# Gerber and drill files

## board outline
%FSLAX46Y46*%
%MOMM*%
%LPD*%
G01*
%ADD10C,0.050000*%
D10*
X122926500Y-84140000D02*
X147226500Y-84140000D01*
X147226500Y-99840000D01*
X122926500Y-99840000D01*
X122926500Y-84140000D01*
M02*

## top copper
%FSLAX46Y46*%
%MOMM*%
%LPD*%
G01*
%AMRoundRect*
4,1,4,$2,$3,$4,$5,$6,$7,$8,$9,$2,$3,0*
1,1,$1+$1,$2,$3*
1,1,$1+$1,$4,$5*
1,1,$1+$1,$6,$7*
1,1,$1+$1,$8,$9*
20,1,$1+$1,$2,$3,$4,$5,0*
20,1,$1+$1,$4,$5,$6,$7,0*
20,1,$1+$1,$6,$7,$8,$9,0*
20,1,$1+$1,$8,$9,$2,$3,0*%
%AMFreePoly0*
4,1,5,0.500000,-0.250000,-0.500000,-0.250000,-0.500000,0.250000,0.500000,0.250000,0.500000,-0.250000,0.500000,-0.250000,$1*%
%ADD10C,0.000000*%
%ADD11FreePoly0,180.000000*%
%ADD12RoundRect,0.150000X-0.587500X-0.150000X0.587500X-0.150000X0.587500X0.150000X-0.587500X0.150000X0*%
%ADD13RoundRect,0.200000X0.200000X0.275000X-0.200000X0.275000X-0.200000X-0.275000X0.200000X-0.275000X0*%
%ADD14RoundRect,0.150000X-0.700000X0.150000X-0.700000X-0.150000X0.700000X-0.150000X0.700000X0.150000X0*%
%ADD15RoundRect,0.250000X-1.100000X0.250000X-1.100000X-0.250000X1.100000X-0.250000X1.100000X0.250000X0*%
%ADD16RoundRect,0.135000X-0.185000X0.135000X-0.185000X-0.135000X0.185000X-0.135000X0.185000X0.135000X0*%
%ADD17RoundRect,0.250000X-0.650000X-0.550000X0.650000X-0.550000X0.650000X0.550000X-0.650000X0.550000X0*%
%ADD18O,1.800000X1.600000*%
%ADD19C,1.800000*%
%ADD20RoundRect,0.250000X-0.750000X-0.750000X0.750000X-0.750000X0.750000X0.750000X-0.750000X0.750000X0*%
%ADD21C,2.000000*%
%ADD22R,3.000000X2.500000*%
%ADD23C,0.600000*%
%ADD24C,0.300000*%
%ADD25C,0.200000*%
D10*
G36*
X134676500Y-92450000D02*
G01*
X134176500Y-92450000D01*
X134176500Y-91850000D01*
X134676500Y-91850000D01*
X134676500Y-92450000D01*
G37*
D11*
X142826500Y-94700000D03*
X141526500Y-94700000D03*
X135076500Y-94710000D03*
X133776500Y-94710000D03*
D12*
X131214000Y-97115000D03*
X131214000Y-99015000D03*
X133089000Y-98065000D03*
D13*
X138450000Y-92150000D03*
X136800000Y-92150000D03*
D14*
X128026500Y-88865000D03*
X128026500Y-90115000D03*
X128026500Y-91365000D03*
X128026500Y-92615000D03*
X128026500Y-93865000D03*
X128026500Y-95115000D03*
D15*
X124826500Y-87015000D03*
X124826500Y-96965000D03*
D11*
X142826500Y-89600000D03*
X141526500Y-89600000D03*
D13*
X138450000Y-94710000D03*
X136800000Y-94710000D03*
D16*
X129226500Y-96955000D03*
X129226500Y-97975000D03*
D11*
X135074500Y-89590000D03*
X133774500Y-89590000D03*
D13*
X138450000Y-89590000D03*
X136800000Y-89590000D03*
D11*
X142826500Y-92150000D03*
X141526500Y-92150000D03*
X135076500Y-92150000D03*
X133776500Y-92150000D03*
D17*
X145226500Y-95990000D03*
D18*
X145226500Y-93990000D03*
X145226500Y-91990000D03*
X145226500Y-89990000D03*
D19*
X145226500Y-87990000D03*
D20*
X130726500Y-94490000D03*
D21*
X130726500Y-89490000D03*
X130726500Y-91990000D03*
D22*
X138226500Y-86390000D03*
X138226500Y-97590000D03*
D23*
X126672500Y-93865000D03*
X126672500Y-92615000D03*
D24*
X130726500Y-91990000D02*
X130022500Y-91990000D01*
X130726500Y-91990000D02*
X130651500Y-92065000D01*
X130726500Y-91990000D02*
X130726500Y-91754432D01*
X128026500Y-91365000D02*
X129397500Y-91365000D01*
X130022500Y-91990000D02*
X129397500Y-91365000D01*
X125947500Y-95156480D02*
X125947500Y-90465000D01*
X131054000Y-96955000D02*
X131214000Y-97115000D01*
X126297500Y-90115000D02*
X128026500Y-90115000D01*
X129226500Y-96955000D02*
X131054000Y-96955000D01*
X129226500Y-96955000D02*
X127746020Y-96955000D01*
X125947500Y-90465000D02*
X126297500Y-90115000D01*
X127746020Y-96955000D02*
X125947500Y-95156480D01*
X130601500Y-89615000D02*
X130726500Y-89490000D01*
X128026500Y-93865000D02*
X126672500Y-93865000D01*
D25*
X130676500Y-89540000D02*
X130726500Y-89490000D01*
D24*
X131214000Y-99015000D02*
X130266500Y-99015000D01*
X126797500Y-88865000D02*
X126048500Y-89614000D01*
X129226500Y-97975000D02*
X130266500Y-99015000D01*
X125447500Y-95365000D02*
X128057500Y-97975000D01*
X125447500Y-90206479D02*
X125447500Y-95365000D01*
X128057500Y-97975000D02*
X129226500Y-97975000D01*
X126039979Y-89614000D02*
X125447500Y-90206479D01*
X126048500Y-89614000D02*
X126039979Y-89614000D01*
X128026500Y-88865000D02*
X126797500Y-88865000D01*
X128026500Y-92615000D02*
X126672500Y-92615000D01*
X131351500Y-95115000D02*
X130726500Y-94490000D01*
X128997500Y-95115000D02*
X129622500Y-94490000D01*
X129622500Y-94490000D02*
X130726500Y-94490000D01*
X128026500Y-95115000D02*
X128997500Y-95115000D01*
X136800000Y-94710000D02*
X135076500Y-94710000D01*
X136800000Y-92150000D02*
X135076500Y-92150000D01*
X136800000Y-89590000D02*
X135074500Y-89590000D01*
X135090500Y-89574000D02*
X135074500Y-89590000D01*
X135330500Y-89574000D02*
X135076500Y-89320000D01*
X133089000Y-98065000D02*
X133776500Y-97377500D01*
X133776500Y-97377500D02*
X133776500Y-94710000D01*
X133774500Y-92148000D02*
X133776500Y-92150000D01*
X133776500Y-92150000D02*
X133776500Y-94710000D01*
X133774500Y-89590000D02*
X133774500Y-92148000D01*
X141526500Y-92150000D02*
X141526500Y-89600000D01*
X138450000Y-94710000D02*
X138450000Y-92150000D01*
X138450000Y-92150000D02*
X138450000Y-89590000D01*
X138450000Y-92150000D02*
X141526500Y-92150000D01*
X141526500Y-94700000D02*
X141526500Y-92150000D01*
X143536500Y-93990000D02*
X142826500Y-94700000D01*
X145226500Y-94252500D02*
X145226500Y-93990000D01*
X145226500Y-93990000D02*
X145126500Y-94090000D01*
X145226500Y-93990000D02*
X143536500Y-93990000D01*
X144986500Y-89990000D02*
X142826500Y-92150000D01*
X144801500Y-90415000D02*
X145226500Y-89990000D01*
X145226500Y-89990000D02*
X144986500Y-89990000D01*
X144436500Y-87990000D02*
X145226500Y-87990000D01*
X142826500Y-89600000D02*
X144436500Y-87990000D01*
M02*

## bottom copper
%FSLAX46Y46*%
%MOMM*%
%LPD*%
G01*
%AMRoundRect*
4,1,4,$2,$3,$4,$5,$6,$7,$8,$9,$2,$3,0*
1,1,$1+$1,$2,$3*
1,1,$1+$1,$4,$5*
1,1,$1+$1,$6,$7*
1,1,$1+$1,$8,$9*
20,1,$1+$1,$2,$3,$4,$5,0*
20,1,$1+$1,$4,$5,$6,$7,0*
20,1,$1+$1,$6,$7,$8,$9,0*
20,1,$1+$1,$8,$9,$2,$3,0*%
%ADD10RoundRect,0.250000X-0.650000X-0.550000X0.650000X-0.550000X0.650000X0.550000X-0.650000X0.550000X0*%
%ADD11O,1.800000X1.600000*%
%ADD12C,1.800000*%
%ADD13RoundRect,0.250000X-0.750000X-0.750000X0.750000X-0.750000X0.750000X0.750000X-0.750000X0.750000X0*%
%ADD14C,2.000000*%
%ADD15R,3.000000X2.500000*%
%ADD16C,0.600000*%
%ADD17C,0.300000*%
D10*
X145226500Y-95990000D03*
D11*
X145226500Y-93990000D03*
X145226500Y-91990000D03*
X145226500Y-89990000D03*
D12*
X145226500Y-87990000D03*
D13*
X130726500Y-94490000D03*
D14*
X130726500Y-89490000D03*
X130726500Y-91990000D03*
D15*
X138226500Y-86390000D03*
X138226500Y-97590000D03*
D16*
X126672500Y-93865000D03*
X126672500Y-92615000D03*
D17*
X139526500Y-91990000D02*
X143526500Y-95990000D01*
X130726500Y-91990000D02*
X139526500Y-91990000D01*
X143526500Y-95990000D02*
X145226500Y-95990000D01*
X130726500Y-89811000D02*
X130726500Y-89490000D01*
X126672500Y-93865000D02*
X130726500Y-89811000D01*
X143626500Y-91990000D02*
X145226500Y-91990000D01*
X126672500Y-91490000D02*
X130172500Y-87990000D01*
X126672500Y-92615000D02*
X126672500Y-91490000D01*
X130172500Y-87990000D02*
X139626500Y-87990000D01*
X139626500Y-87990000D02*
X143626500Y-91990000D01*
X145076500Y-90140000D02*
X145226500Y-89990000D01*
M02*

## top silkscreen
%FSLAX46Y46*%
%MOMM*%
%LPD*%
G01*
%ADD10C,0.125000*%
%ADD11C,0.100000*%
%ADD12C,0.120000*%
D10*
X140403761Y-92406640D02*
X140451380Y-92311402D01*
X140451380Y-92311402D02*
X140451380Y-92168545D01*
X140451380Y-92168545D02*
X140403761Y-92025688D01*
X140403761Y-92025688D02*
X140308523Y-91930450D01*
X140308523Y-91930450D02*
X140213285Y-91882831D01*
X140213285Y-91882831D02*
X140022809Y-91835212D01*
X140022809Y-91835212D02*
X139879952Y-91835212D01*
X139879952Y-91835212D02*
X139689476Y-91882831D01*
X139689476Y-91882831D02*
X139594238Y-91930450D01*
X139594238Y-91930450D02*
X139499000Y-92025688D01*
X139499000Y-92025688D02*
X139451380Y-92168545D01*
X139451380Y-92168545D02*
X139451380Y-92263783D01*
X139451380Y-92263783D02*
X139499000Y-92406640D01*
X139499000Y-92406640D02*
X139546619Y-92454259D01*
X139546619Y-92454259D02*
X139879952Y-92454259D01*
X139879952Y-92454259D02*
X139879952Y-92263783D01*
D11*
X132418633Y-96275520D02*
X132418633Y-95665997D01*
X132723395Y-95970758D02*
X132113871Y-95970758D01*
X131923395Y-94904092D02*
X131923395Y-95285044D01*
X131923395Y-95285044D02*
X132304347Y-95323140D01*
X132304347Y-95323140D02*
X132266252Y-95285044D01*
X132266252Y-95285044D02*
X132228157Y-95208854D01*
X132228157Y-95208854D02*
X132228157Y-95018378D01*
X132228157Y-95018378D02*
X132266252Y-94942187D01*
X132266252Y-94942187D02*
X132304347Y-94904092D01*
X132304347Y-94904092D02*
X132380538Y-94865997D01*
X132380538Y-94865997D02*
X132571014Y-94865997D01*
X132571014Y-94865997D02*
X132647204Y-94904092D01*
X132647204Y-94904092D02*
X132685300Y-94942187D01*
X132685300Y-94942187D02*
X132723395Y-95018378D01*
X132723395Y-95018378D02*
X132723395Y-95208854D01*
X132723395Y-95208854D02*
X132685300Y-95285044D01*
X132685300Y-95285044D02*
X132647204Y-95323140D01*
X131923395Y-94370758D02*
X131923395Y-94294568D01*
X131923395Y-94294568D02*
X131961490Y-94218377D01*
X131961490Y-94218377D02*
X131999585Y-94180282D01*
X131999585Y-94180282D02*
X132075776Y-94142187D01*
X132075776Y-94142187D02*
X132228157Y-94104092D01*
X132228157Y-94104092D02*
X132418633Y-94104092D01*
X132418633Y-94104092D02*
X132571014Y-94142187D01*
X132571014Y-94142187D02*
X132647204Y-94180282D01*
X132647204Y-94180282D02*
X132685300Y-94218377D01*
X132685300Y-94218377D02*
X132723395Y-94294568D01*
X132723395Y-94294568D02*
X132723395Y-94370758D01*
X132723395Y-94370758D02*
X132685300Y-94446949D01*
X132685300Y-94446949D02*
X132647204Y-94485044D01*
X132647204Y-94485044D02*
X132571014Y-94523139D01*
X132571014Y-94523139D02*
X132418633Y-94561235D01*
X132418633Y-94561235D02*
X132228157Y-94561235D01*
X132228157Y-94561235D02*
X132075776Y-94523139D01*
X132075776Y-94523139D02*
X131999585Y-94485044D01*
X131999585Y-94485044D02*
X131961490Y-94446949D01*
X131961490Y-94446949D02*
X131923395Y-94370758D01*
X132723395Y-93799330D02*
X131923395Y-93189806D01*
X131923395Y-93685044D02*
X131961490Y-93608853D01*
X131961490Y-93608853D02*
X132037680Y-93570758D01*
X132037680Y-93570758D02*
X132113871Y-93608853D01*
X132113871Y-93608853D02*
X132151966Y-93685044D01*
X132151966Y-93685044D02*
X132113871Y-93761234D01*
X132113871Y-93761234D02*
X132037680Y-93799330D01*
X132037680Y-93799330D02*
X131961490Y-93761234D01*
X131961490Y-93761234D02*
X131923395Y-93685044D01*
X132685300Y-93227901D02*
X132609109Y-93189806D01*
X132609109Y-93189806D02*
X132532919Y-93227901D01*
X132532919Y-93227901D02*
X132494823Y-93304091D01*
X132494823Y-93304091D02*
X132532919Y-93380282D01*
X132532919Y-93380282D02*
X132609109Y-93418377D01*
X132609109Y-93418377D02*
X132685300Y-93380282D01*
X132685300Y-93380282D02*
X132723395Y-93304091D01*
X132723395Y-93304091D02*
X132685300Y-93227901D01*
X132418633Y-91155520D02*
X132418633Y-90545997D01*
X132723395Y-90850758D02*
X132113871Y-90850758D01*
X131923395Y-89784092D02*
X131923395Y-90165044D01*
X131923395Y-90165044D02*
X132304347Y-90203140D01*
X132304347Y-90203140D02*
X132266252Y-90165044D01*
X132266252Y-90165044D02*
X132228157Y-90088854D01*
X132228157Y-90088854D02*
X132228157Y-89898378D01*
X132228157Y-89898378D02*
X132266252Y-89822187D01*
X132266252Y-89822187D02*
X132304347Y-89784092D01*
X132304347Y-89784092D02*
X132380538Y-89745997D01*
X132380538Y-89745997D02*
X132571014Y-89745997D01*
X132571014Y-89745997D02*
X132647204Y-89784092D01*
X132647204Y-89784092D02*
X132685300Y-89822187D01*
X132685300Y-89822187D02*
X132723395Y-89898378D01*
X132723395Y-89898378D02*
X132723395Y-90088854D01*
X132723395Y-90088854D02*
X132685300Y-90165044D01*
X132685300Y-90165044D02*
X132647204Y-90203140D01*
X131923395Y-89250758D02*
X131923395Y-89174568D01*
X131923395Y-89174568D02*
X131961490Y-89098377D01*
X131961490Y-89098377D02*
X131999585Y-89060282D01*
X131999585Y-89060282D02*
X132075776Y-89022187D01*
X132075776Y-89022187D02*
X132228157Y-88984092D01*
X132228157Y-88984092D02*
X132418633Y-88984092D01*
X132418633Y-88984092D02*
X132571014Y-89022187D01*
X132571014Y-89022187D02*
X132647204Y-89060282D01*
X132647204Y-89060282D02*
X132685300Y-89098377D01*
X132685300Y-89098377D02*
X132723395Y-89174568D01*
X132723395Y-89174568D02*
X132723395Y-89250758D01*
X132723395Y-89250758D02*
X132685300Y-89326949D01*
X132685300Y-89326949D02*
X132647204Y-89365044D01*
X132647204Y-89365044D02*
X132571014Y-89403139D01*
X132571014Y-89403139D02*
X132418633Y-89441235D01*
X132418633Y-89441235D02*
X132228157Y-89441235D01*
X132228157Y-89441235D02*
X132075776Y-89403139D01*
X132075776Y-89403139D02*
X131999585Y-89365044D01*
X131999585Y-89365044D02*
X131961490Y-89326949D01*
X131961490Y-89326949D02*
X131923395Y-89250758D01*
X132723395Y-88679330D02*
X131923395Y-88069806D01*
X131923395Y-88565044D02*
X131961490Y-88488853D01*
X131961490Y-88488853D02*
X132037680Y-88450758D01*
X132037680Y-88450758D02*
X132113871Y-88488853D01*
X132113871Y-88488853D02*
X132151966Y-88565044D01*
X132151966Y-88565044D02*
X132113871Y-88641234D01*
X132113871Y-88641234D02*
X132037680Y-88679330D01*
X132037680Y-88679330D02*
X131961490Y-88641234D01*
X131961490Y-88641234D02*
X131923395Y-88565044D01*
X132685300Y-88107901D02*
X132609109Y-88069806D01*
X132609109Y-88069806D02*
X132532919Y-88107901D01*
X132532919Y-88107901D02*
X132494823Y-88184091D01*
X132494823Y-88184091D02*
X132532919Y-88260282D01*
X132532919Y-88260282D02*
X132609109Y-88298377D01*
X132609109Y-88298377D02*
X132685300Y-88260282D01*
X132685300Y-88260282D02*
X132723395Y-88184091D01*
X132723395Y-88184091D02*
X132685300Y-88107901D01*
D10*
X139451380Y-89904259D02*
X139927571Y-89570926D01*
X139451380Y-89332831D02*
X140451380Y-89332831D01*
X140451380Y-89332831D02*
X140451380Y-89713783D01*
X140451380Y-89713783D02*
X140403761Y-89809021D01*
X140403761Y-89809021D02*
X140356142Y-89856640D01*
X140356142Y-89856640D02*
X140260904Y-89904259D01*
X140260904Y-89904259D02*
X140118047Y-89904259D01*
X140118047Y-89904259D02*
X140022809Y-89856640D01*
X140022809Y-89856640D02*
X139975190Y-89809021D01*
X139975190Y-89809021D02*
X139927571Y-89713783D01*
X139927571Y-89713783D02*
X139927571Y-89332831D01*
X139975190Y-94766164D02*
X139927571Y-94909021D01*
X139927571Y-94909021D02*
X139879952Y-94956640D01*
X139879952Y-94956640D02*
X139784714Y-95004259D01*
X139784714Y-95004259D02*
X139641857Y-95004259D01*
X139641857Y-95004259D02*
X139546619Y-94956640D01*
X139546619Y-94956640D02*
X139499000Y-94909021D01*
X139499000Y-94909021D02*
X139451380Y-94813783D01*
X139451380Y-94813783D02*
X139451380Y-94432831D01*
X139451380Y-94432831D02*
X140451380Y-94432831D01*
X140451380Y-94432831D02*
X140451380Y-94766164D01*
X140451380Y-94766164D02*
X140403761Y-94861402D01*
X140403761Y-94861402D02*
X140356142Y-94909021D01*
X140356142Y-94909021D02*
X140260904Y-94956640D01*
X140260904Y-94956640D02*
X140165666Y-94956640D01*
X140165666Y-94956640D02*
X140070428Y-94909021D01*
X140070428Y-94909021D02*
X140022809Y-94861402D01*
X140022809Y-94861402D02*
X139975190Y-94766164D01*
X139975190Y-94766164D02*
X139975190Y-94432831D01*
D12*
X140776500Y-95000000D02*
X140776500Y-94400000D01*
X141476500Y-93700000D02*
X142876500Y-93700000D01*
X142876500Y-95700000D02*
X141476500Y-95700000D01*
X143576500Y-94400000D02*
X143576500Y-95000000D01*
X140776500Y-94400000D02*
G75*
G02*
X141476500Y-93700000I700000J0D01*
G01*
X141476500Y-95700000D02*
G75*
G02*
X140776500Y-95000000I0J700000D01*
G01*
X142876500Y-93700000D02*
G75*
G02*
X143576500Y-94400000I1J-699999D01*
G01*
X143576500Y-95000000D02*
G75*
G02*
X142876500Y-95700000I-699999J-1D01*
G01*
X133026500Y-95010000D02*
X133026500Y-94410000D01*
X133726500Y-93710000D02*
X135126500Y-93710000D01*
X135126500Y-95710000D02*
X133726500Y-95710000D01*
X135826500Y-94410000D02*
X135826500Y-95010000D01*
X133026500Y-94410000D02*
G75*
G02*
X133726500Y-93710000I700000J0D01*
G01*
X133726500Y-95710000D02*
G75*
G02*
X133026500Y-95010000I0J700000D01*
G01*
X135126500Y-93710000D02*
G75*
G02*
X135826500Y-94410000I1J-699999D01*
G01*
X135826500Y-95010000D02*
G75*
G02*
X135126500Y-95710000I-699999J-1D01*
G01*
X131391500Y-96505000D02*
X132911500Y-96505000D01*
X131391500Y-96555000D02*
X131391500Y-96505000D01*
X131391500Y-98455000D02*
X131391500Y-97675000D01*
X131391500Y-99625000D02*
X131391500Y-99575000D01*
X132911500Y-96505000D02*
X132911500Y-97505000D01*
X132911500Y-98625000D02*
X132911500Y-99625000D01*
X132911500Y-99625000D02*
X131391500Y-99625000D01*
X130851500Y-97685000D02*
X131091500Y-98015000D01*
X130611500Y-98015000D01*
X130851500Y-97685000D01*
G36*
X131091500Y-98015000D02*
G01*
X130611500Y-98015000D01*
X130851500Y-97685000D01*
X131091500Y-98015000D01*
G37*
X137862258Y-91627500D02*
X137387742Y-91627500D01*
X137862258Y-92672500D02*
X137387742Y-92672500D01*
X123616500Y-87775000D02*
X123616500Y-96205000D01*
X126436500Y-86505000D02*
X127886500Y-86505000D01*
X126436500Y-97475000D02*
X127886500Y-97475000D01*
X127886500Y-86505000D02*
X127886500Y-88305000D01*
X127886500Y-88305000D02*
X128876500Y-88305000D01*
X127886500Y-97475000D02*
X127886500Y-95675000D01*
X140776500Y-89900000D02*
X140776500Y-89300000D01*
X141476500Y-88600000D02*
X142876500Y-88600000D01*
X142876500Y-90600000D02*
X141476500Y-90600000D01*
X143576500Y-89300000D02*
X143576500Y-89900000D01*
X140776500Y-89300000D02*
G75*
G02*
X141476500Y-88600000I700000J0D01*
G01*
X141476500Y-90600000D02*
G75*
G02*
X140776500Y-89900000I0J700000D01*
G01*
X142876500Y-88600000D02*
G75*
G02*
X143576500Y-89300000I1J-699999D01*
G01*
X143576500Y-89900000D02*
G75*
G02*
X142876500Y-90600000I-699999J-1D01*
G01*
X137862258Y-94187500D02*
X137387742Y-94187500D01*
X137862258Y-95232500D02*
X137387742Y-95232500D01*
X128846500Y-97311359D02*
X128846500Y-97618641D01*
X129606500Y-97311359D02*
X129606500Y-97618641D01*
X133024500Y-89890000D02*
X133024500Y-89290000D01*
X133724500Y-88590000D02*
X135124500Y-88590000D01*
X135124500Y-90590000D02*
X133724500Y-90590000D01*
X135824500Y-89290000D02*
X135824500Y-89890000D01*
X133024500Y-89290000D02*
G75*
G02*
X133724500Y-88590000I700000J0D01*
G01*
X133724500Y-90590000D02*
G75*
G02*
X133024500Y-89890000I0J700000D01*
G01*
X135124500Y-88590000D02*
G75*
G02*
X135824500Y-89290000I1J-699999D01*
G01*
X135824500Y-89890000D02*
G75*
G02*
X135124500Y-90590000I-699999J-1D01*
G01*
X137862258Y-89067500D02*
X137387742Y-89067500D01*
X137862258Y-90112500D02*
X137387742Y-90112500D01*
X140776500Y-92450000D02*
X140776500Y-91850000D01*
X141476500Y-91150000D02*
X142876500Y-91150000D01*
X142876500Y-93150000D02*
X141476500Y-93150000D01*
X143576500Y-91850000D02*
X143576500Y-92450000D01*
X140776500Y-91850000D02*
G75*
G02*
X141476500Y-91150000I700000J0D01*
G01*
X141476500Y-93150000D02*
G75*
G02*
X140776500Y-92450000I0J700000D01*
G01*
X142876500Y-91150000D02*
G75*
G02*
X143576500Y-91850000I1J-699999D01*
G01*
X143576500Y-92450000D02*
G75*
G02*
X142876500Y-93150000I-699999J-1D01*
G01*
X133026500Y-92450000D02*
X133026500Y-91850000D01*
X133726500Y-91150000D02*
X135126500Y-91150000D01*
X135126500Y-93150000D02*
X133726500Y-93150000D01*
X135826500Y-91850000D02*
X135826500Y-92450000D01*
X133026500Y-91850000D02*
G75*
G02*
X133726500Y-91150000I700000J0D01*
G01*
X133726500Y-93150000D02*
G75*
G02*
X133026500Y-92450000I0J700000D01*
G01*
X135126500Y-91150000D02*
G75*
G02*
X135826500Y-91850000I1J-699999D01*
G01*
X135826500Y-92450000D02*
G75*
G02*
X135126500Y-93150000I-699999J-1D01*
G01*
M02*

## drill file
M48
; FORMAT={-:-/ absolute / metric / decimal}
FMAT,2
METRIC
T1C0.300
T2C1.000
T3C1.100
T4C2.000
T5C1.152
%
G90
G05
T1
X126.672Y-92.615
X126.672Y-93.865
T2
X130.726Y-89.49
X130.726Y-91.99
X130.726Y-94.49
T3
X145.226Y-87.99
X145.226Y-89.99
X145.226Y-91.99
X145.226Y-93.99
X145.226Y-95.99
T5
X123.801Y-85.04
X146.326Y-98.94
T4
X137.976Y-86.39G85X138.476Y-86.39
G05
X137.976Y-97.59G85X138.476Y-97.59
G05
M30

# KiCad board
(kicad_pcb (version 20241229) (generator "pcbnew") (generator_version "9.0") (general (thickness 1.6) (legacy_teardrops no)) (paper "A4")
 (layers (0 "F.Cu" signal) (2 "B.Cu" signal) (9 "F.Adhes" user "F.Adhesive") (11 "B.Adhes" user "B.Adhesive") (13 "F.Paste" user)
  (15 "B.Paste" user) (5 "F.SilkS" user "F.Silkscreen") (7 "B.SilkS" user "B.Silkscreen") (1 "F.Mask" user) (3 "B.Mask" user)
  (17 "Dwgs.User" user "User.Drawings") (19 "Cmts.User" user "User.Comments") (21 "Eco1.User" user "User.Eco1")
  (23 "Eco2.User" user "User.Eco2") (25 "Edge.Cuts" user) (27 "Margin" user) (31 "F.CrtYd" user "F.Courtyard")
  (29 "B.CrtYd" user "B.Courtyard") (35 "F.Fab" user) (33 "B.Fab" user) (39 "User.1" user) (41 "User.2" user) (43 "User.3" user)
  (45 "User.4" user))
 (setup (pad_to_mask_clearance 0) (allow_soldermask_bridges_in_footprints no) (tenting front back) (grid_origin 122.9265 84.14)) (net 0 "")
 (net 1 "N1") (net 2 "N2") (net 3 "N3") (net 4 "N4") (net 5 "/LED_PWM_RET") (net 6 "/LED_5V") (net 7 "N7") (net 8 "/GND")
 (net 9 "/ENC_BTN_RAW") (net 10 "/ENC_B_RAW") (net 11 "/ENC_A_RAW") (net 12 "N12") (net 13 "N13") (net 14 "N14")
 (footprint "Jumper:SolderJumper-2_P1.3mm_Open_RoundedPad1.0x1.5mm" (layer "F.Cu") (at 142.1765 94.7 180)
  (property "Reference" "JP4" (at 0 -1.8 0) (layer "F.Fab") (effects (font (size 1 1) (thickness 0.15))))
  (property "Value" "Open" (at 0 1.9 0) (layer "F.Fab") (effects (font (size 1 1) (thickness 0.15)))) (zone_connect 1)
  (fp_line (start 1.4 -0.3) (end 1.4 0.3) (stroke (width 0.12) (type solid)) (layer "F.SilkS"))
  (fp_line (start 0.7 1) (end -0.7 1) (stroke (width 0.12) (type solid)) (layer "F.SilkS"))
  (fp_line (start -0.7 -1) (end 0.7 -1) (stroke (width 0.12) (type solid)) (layer "F.SilkS"))
  (fp_line (start -1.4 0.3) (end -1.4 -0.3) (stroke (width 0.12) (type solid)) (layer "F.SilkS"))
  (fp_arc (start 1.4 0.3) (mid 1.194975 0.794975) (end 0.7 1) (stroke (width 0.12) (type solid)) (layer "F.SilkS"))
  (fp_arc (start 0.7 -1) (mid 1.194975 -0.794975) (end 1.4 -0.3) (stroke (width 0.12) (type solid)) (layer "F.SilkS"))
  (fp_arc (start -0.7 1) (mid -1.194975 0.794975) (end -1.4 0.3) (stroke (width 0.12) (type solid)) (layer "F.SilkS"))
  (fp_arc (start -1.4 -0.3) (mid -1.194975 -0.794975) (end -0.7 -1) (stroke (width 0.12) (type solid)) (layer "F.SilkS"))
  (pad "1" smd custom (at -0.65 0 180) (size 1 0.5) (layers "F.Cu" "F.Mask") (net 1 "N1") (zone_connect 2) (thermal_bridge_angle 45)
   (options (clearance outline) (anchor rect)) (primitives))
  (pad "2" smd custom (at 0.65 0 180) (size 1 0.5) (layers "F.Cu" "F.Mask") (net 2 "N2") (zone_connect 2) (thermal_bridge_angle 45)
   (options (clearance outline) (anchor rect)) (primitives)))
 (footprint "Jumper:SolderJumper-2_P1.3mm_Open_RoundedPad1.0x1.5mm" (layer "F.Cu") (at 134.4265 94.71 180)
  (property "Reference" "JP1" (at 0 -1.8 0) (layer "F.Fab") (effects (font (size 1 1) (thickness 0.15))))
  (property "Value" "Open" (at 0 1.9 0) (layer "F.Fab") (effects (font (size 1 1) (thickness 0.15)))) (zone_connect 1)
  (fp_line (start 1.4 -0.3) (end 1.4 0.3) (stroke (width 0.12) (type solid)) (layer "F.SilkS"))
  (fp_line (start 0.7 1) (end -0.7 1) (stroke (width 0.12) (type solid)) (layer "F.SilkS"))
  (fp_line (start -0.7 -1) (end 0.7 -1) (stroke (width 0.12) (type solid)) (layer "F.SilkS"))
  (fp_line (start -1.4 0.3) (end -1.4 -0.3) (stroke (width 0.12) (type solid)) (layer "F.SilkS"))
  (fp_arc (start 1.4 0.3) (mid 1.194975 0.794975) (end 0.7 1) (stroke (width 0.12) (type solid)) (layer "F.SilkS"))
  (fp_arc (start 0.7 -1) (mid 1.194975 -0.794975) (end 1.4 -0.3) (stroke (width 0.12) (type solid)) (layer "F.SilkS"))
  (fp_arc (start -0.7 1) (mid -1.194975 0.794975) (end -1.4 0.3) (stroke (width 0.12) (type solid)) (layer "F.SilkS"))
  (fp_arc (start -1.4 -0.3) (mid -1.194975 -0.794975) (end -0.7 -1) (stroke (width 0.12) (type solid)) (layer "F.SilkS"))
  (pad "1" smd custom (at -0.65 0 180) (size 1 0.5) (layers "F.Cu" "F.Mask") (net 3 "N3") (zone_connect 2) (thermal_bridge_angle 45)
   (options (clearance outline) (anchor rect)) (primitives))
  (pad "2" smd custom (at 0.65 0 180) (size 1 0.5) (layers "F.Cu" "F.Mask") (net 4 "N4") (zone_connect 2) (thermal_bridge_angle 45)
   (options (clearance outline) (anchor rect)) (primitives)))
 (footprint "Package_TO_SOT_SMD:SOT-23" (layer "F.Cu") (at 132.1515 98.065)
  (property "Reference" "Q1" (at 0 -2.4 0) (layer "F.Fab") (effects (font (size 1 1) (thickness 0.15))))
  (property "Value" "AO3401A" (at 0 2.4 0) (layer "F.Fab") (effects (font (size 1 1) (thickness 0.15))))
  (fp_line (start -0.76 -1.56) (end 0.76 -1.56) (stroke (width 0.12) (type solid)) (layer "F.SilkS"))
  (fp_line (start -0.76 -1.51) (end -0.76 -1.56) (stroke (width 0.12) (type solid)) (layer "F.SilkS"))
  (fp_line (start -0.76 0.39) (end -0.76 -0.39) (stroke (width 0.12) (type solid)) (layer "F.SilkS"))
  (fp_line (start -0.76 1.56) (end -0.76 1.51) (stroke (width 0.12) (type solid)) (layer "F.SilkS"))
  (fp_line (start 0.76 -1.56) (end 0.76 -0.56) (stroke (width 0.12) (type solid)) (layer "F.SilkS"))
  (fp_line (start 0.76 0.56) (end 0.76 1.56) (stroke (width 0.12) (type solid)) (layer "F.SilkS"))
  (fp_line (start 0.76 1.56) (end -0.76 1.56) (stroke (width 0.12) (type solid)) (layer "F.SilkS"))
  (fp_poly (pts (xy -1.3 -0.38) (xy -1.06 -0.05) (xy -1.54 -0.05)) (stroke (width 0.12) (type solid)) (fill yes) (layer "F.SilkS"))
  (pad "1" smd roundrect (at -0.9375 -0.95) (size 1.475 0.6) (layers "F.Cu" "F.Mask" "F.Paste") (roundrect_rratio 0.25)
   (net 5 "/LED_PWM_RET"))
  (pad "2" smd roundrect (at -0.9375 0.95) (size 1.475 0.6) (layers "F.Cu" "F.Mask" "F.Paste") (roundrect_rratio 0.25) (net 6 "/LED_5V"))
  (pad "3" smd roundrect (at 0.9375 0) (size 1.475 0.6) (layers "F.Cu" "F.Mask" "F.Paste") (roundrect_rratio 0.25) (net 4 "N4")))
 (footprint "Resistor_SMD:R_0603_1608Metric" (layer "F.Cu") (at 137.625 92.15 180)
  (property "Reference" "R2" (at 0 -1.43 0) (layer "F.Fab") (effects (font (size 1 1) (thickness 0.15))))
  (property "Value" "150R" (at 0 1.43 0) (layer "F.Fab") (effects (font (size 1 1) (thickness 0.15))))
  (fp_line (start -0.237258 0.5225) (end 0.237258 0.5225) (stroke (width 0.12) (type solid)) (layer "F.SilkS"))
  (fp_line (start -0.237258 -0.5225) (end 0.237258 -0.5225) (stroke (width 0.12) (type solid)) (layer "F.SilkS"))
  (pad "1" smd roundrect (at -0.825 0 180) (size 0.8 0.95) (layers "F.Cu" "F.Mask" "F.Paste") (roundrect_rratio 0.25) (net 2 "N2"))
  (pad "2" smd roundrect (at 0.825 0 180) (size 0.8 0.95) (layers "F.Cu" "F.Mask" "F.Paste") (roundrect_rratio 0.25) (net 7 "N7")))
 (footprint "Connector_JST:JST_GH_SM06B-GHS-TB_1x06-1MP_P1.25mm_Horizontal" (layer "F.Cu") (at 126.1765 91.99 -90)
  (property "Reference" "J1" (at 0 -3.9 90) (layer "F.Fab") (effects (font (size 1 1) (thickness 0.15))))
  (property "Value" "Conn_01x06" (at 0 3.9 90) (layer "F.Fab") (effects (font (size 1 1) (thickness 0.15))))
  (fp_line (start -4.215 2.56) (end 4.215 2.56) (stroke (width 0.12) (type solid)) (layer "F.SilkS"))
  (fp_line (start -5.485 -0.26) (end -5.485 -1.71) (stroke (width 0.12) (type solid)) (layer "F.SilkS"))
  (fp_line (start 5.485 -0.26) (end 5.485 -1.71) (stroke (width 0.12) (type solid)) (layer "F.SilkS"))
  (fp_line (start -5.485 -1.71) (end -3.685 -1.71) (stroke (width 0.12) (type solid)) (layer "F.SilkS"))
  (fp_line (start -3.685 -1.71) (end -3.685 -2.7) (stroke (width 0.12) (type solid)) (layer "F.SilkS"))
  (fp_line (start 5.485 -1.71) (end 3.685 -1.71) (stroke (width 0.12) (type solid)) (layer "F.SilkS"))
  (pad "1" smd roundrect (at -3.125 -1.85 270) (size 0.6 1.7) (layers "F.Cu" "F.Mask" "F.Paste") (roundrect_rratio 0.25) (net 6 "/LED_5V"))
  (pad "2" smd roundrect (at -1.875 -1.85 270) (size 0.6 1.7) (layers "F.Cu" "F.Mask" "F.Paste") (roundrect_rratio 0.25)
   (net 5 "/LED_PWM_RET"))
  (pad "3" smd roundrect (at -0.625 -1.85 270) (size 0.6 1.7) (layers "F.Cu" "F.Mask" "F.Paste") (roundrect_rratio 0.25) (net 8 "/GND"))
  (pad "4" smd roundrect (at 0.625 -1.85 270) (size 0.6 1.7) (layers "F.Cu" "F.Mask" "F.Paste") (roundrect_rratio 0.25)
   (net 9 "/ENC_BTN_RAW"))
  (pad "5" smd roundrect (at 1.875 -1.85 270) (size 0.6 1.7) (layers "F.Cu" "F.Mask" "F.Paste") (roundrect_rratio 0.25)
   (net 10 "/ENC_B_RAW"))
  (pad "6" smd roundrect (at 3.125 -1.85 270) (size 0.6 1.7) (layers "F.Cu" "F.Mask" "F.Paste") (roundrect_rratio 0.25)
   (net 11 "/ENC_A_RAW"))
  (pad "MP" smd roundrect (at -4.975 1.35 270) (size 1 2.7) (layers "F.Cu" "F.Mask" "F.Paste") (roundrect_rratio 0.25))
  (pad "MP" smd roundrect (at 4.975 1.35 270) (size 1 2.7) (layers "F.Cu" "F.Mask" "F.Paste") (roundrect_rratio 0.25)))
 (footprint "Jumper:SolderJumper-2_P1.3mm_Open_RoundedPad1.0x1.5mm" (layer "F.Cu") (at 142.1765 89.6 180)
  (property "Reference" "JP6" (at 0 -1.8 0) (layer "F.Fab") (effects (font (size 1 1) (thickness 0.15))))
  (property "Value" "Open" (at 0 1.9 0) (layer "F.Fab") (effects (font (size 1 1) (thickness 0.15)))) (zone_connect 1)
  (fp_line (start 1.4 -0.3) (end 1.4 0.3) (stroke (width 0.12) (type solid)) (layer "F.SilkS"))
  (fp_line (start 0.7 1) (end -0.7 1) (stroke (width 0.12) (type solid)) (layer "F.SilkS"))
  (fp_line (start -0.7 -1) (end 0.7 -1) (stroke (width 0.12) (type solid)) (layer "F.SilkS"))
  (fp_line (start -1.4 0.3) (end -1.4 -0.3) (stroke (width 0.12) (type solid)) (layer "F.SilkS"))
  (fp_arc (start 1.4 0.3) (mid 1.194975 0.794975) (end 0.7 1) (stroke (width 0.12) (type solid)) (layer "F.SilkS"))
  (fp_arc (start 0.7 -1) (mid 1.194975 -0.794975) (end 1.4 -0.3) (stroke (width 0.12) (type solid)) (layer "F.SilkS"))
  (fp_arc (start -0.7 1) (mid -1.194975 0.794975) (end -1.4 0.3) (stroke (width 0.12) (type solid)) (layer "F.SilkS"))
  (fp_arc (start -1.4 -0.3) (mid -1.194975 -0.794975) (end -0.7 -1) (stroke (width 0.12) (type solid)) (layer "F.SilkS"))
  (pad "1" smd custom (at -0.65 0 180) (size 1 0.5) (layers "F.Cu" "F.Mask") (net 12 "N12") (zone_connect 2) (thermal_bridge_angle 45)
   (options (clearance outline) (anchor rect)) (primitives))
  (pad "2" smd custom (at 0.65 0 180) (size 1 0.5) (layers "F.Cu" "F.Mask") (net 2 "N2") (zone_connect 2) (thermal_bridge_angle 45)
   (options (clearance outline) (anchor rect)) (primitives)))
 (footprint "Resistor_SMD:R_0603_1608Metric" (layer "F.Cu") (at 137.625 94.71 180)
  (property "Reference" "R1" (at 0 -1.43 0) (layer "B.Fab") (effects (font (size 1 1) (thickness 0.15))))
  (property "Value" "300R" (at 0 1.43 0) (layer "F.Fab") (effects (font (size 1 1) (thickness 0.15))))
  (fp_line (start -0.237258 0.5225) (end 0.237258 0.5225) (stroke (width 0.12) (type solid)) (layer "F.SilkS"))
  (fp_line (start -0.237258 -0.5225) (end 0.237258 -0.5225) (stroke (width 0.12) (type solid)) (layer "F.SilkS"))
  (pad "1" smd roundrect (at -0.825 0 180) (size 0.8 0.95) (layers "F.Cu" "F.Mask" "F.Paste") (roundrect_rratio 0.25) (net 2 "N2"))
  (pad "2" smd roundrect (at 0.825 0 180) (size 0.8 0.95) (layers "F.Cu" "F.Mask" "F.Paste") (roundrect_rratio 0.25) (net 3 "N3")))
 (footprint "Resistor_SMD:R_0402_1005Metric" (layer "F.Cu") (at 129.2265 97.465 -90)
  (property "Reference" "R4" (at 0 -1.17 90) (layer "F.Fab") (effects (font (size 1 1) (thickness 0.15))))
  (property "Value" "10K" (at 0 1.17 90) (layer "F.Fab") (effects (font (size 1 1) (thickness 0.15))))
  (fp_line (start -0.153641 0.38) (end 0.153641 0.38) (stroke (width 0.12) (type solid)) (layer "F.SilkS"))
  (fp_line (start -0.153641 -0.38) (end 0.153641 -0.38) (stroke (width 0.12) (type solid)) (layer "F.SilkS"))
  (pad "1" smd roundrect (at -0.51 0 270) (size 0.54 0.64) (layers "F.Cu" "F.Mask" "F.Paste") (roundrect_rratio 0.25) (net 5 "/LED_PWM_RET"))
  (pad "2" smd roundrect (at 0.51 0 270) (size 0.54 0.64) (layers "F.Cu" "F.Mask" "F.Paste") (roundrect_rratio 0.25) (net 6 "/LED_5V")))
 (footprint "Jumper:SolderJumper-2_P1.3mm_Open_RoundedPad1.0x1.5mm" (layer "F.Cu") (at 134.4245 89.59 180)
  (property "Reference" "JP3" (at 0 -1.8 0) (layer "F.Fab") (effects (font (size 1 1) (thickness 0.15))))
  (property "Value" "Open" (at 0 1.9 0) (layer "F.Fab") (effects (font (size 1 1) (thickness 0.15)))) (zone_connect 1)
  (fp_line (start 1.4 -0.3) (end 1.4 0.3) (stroke (width 0.12) (type solid)) (layer "F.SilkS"))
  (fp_line (start 0.7 1) (end -0.7 1) (stroke (width 0.12) (type solid)) (layer "F.SilkS"))
  (fp_line (start -0.7 -1) (end 0.7 -1) (stroke (width 0.12) (type solid)) (layer "F.SilkS"))
  (fp_line (start -1.4 0.3) (end -1.4 -0.3) (stroke (width 0.12) (type solid)) (layer "F.SilkS"))
  (fp_arc (start 1.4 0.3) (mid 1.194975 0.794975) (end 0.7 1) (stroke (width 0.12) (type solid)) (layer "F.SilkS"))
  (fp_arc (start 0.7 -1) (mid 1.194975 -0.794975) (end 1.4 -0.3) (stroke (width 0.12) (type solid)) (layer "F.SilkS"))
  (fp_arc (start -0.7 1) (mid -1.194975 0.794975) (end -1.4 0.3) (stroke (width 0.12) (type solid)) (layer "F.SilkS"))
  (fp_arc (start -1.4 -0.3) (mid -1.194975 -0.794975) (end -0.7 -1) (stroke (width 0.12) (type solid)) (layer "F.SilkS"))
  (pad "1" smd custom (at -0.65 0 180) (size 1 0.5) (layers "F.Cu" "F.Mask") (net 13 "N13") (zone_connect 2) (thermal_bridge_angle 45)
   (options (clearance outline) (anchor rect)) (primitives))
  (pad "2" smd custom (at 0.65 0 180) (size 1 0.5) (layers "F.Cu" "F.Mask") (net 4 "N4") (zone_connect 2) (thermal_bridge_angle 45)
   (options (clearance outline) (anchor rect)) (primitives)))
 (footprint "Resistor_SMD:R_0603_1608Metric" (layer "F.Cu") (at 137.625 89.59 180)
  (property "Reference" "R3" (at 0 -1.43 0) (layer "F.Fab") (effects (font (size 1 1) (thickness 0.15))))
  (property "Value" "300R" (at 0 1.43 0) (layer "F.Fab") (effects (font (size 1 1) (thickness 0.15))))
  (fp_line (start -0.237258 0.5225) (end 0.237258 0.5225) (stroke (width 0.12) (type solid)) (layer "F.SilkS"))
  (fp_line (start -0.237258 -0.5225) (end 0.237258 -0.5225) (stroke (width 0.12) (type solid)) (layer "F.SilkS"))
  (pad "1" smd roundrect (at -0.825 0 180) (size 0.8 0.95) (layers "F.Cu" "F.Mask" "F.Paste") (roundrect_rratio 0.25) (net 2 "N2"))
  (pad "2" smd roundrect (at 0.825 0 180) (size 0.8 0.95) (layers "F.Cu" "F.Mask" "F.Paste") (roundrect_rratio 0.25) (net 13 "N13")))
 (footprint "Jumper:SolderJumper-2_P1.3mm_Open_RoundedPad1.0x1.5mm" (layer "F.Cu") (at 142.1765 92.15 180)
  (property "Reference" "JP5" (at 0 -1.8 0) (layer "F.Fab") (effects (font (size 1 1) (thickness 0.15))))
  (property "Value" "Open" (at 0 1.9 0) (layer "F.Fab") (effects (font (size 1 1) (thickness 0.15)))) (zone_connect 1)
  (fp_line (start 1.4 -0.3) (end 1.4 0.3) (stroke (width 0.12) (type solid)) (layer "F.SilkS"))
  (fp_line (start 0.7 1) (end -0.7 1) (stroke (width 0.12) (type solid)) (layer "F.SilkS"))
  (fp_line (start -0.7 -1) (end 0.7 -1) (stroke (width 0.12) (type solid)) (layer "F.SilkS"))
  (fp_line (start -1.4 0.3) (end -1.4 -0.3) (stroke (width 0.12) (type solid)) (layer "F.SilkS"))
  (fp_arc (start 1.4 0.3) (mid 1.194975 0.794975) (end 0.7 1) (stroke (width 0.12) (type solid)) (layer "F.SilkS"))
  (fp_arc (start 0.7 -1) (mid 1.194975 -0.794975) (end 1.4 -0.3) (stroke (width 0.12) (type solid)) (layer "F.SilkS"))
  (fp_arc (start -0.7 1) (mid -1.194975 0.794975) (end -1.4 0.3) (stroke (width 0.12) (type solid)) (layer "F.SilkS"))
  (fp_arc (start -1.4 -0.3) (mid -1.194975 -0.794975) (end -0.7 -1) (stroke (width 0.12) (type solid)) (layer "F.SilkS"))
  (pad "1" smd custom (at -0.65 0 180) (size 1 0.5) (layers "F.Cu" "F.Mask") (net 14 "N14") (zone_connect 2) (thermal_bridge_angle 45)
   (options (clearance outline) (anchor rect)) (primitives))
  (pad "2" smd custom (at 0.65 0 180) (size 1 0.5) (layers "F.Cu" "F.Mask") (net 2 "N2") (zone_connect 2) (thermal_bridge_angle 45)
   (options (clearance outline) (anchor rect)) (primitives)))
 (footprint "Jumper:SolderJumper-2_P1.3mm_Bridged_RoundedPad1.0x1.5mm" (layer "F.Cu") (at 134.4265 92.15 180)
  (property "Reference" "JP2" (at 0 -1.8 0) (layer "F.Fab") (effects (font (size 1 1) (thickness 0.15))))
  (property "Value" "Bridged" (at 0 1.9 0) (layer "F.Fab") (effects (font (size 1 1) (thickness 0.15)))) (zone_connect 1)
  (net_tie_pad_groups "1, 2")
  (fp_poly (pts (xy 0.25 -0.3) (xy -0.25 -0.3) (xy -0.25 0.3) (xy 0.25 0.3)) (stroke (width 0) (type solid)) (fill yes) (layer "F.Cu"))
  (fp_line (start 1.4 -0.3) (end 1.4 0.3) (stroke (width 0.12) (type solid)) (layer "F.SilkS"))
  (fp_line (start 0.7 1) (end -0.7 1) (stroke (width 0.12) (type solid)) (layer "F.SilkS"))
  (fp_line (start -0.7 -1) (end 0.7 -1) (stroke (width 0.12) (type solid)) (layer "F.SilkS"))
  (fp_line (start -1.4 0.3) (end -1.4 -0.3) (stroke (width 0.12) (type solid)) (layer "F.SilkS"))
  (fp_arc (start 1.4 0.3) (mid 1.194975 0.794975) (end 0.7 1) (stroke (width 0.12) (type solid)) (layer "F.SilkS"))
  (fp_arc (start 0.7 -1) (mid 1.194975 -0.794975) (end 1.4 -0.3) (stroke (width 0.12) (type solid)) (layer "F.SilkS"))
  (fp_arc (start -0.7 1) (mid -1.194975 0.794975) (end -1.4 0.3) (stroke (width 0.12) (type solid)) (layer "F.SilkS"))
  (fp_arc (start -1.4 -0.3) (mid -1.194975 -0.794975) (end -0.7 -1) (stroke (width 0.12) (type solid)) (layer "F.SilkS"))
  (pad "1" smd custom (at -0.65 0 180) (size 1 0.5) (layers "F.Cu" "F.Mask") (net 7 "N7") (zone_connect 2) (thermal_bridge_angle 45)
   (options (clearance outline) (anchor rect)) (primitives))
  (pad "2" smd custom (at 0.65 0 180) (size 1 0.5) (layers "F.Cu" "F.Mask") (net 4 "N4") (zone_connect 2) (thermal_bridge_angle 45)
   (options (clearance outline) (anchor rect)) (primitives)))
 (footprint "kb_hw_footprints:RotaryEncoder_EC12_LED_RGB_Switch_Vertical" (layer "B.Cu") (at 130.7265 94.49)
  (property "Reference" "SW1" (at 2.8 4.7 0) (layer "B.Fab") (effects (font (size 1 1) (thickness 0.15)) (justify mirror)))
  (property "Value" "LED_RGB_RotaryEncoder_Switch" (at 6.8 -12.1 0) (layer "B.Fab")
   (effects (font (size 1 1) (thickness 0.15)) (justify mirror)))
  (pad "1" thru_hole roundrect (at 14.5 1.5) (size 1.8 1.6) (drill 1.1) (layers "*.Cu" "*.Mask") (remove_unused_layers no)
   (roundrect_rratio 0.15625) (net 8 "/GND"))
  (pad "2" thru_hole oval (at 14.5 -0.5) (size 1.8 1.6) (drill 1.1) (layers "*.Cu" "*.Mask") (remove_unused_layers no) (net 1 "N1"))
  (pad "3" thru_hole oval (at 14.5 -2.5) (size 1.8 1.6) (drill 1.1) (layers "*.Cu" "*.Mask") (remove_unused_layers no)
   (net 9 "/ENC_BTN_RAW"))
  (pad "4" thru_hole oval (at 14.5 -4.5) (size 1.8 1.6) (drill 1.1) (layers "*.Cu" "*.Mask") (remove_unused_layers no) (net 14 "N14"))
  (pad "5" thru_hole circle (at 14.5 -6.5) (size 1.8 1.8) (drill 1.1) (layers "*.Cu" "*.Mask") (remove_unused_layers no) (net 12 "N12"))
  (pad "A" thru_hole roundrect (at 0 0) (size 2 2) (drill 1) (layers "*.Cu" "*.Mask") (remove_unused_layers no) (roundrect_rratio 0.125)
   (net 11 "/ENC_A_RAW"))
  (pad "B" thru_hole circle (at 0 -5) (size 2 2) (drill 1) (layers "*.Cu" "*.Mask") (remove_unused_layers no) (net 10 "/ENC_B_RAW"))
  (pad "C" thru_hole circle (at 0 -2.5) (size 2 2) (drill 1) (layers "*.Cu" "*.Mask") (remove_unused_layers no) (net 8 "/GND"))
  (pad "MP" thru_hole rect (at 7.5 -8.1) (size 3 2.5) (drill oval 2.5 2) (layers "*.Cu" "*.Mask") (remove_unused_layers no))
  (pad "MP" thru_hole rect (at 7.5 3.1) (size 3 2.5) (drill oval 2.5 2) (layers "*.Cu" "*.Mask") (remove_unused_layers no)))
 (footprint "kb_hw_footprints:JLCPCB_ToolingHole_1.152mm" (layer "B.Cu") (at 123.8015 85.04)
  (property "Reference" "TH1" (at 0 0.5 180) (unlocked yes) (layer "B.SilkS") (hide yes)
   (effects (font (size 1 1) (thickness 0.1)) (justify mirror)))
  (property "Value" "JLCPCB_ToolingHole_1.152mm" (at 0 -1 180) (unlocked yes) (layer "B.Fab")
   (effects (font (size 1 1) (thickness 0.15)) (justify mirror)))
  (pad "" np_thru_hole circle (at 0 0) (size 1.152 1.152) (drill 1.152) (layers "*.Cu" "*.Mask") (solder_mask_margin 0.148) (clearance 0.25)
   (thermal_bridge_angle 90)))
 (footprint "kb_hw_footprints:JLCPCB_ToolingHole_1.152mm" (layer "B.Cu") (at 146.3265 98.94)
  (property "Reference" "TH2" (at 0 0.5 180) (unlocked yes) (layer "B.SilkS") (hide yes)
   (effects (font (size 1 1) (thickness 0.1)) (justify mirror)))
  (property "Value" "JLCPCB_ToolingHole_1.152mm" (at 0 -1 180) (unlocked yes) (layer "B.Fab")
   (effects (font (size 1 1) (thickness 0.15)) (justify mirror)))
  (pad "" np_thru_hole circle (at 0 0) (size 1.152 1.152) (drill 1.152) (layers "*.Cu" "*.Mask") (solder_mask_margin 0.148) (clearance 0.25)
   (thermal_bridge_angle 90)))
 (gr_rect (start 122.9265 84.14) (end 147.2265 99.84) (stroke (width 0.05) (type solid)) (fill no) (layer "Edge.Cuts"))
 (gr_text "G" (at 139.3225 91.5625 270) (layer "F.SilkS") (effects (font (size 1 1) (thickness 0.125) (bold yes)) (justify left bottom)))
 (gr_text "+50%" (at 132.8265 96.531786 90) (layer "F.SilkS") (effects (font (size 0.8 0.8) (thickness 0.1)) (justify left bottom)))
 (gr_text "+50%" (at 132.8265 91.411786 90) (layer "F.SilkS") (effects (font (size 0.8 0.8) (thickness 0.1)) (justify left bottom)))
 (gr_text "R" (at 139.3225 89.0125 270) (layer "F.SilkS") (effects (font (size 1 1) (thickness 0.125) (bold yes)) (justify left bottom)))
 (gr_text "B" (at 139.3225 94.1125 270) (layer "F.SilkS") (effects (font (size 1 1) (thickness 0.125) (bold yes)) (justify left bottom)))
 (segment (start 130.7265 91.99) (end 130.0225 91.99) (width 0.3) (layer "F.Cu") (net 8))
 (segment (start 130.7265 91.99) (end 130.6515 92.065) (width 0.3) (layer "F.Cu") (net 8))
 (segment (start 130.7265 91.99) (end 130.7265 91.754432) (width 0.3) (layer "F.Cu") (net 8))
 (segment (start 128.0265 91.365) (end 129.3975 91.365) (width 0.3) (layer "F.Cu") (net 8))
 (segment (start 130.0225 91.99) (end 129.3975 91.365) (width 0.3) (layer "F.Cu") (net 8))
 (segment (start 139.5265 91.99) (end 143.5265 95.99) (width 0.3) (layer "B.Cu") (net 8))
 (segment (start 130.7265 91.99) (end 139.5265 91.99) (width 0.3) (layer "B.Cu") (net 8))
 (segment (start 143.5265 95.99) (end 145.2265 95.99) (width 0.3) (layer "B.Cu") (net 8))
 (segment (start 125.9475 95.15648) (end 125.9475 90.465) (width 0.3) (layer "F.Cu") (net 5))
 (segment (start 131.054 96.955) (end 131.214 97.115) (width 0.3) (layer "F.Cu") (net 5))
 (segment (start 126.2975 90.115) (end 128.0265 90.115) (width 0.3) (layer "F.Cu") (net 5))
 (segment (start 129.2265 96.955) (end 131.054 96.955) (width 0.3) (layer "F.Cu") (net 5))
 (segment (start 129.2265 96.955) (end 127.74602 96.955) (width 0.3) (layer "F.Cu") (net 5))
 (segment (start 125.9475 90.465) (end 126.2975 90.115) (width 0.3) (layer "F.Cu") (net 5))
 (segment (start 127.74602 96.955) (end 125.9475 95.15648) (width 0.3) (layer "F.Cu") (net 5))
 (segment (start 130.6015 89.615) (end 130.7265 89.49) (width 0.3) (layer "F.Cu") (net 10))
 (segment (start 128.0265 93.865) (end 126.6725 93.865) (width 0.3) (layer "F.Cu") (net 10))
 (segment (start 130.6765 89.54) (end 130.7265 89.49) (width 0.2) (layer "F.Cu") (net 10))
 (via (at 126.6725 93.865) (size 0.6) (drill 0.3) (layers "F.Cu" "B.Cu") (free yes) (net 10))
 (segment (start 130.7265 89.811) (end 130.7265 89.49) (width 0.3) (layer "B.Cu") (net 10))
 (segment (start 126.6725 93.865) (end 130.7265 89.811) (width 0.3) (layer "B.Cu") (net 10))
 (segment (start 131.214 99.015) (end 130.2665 99.015) (width 0.3) (layer "F.Cu") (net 6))
 (segment (start 126.7975 88.865) (end 126.0485 89.614) (width 0.3) (layer "F.Cu") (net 6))
 (segment (start 129.2265 97.975) (end 130.2665 99.015) (width 0.3) (layer "F.Cu") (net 6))
 (segment (start 125.4475 95.365) (end 128.0575 97.975) (width 0.3) (layer "F.Cu") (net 6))
 (segment (start 125.4475 90.206479) (end 125.4475 95.365) (width 0.3) (layer "F.Cu") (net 6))
 (segment (start 128.0575 97.975) (end 129.2265 97.975) (width 0.3) (layer "F.Cu") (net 6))
 (segment (start 126.039979 89.614) (end 125.4475 90.206479) (width 0.3) (layer "F.Cu") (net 6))
 (segment (start 126.0485 89.614) (end 126.039979 89.614) (width 0.3) (layer "F.Cu") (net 6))
 (segment (start 128.0265 88.865) (end 126.7975 88.865) (width 0.3) (layer "F.Cu") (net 6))
 (segment (start 128.0265 92.615) (end 126.6725 92.615) (width 0.3) (layer "F.Cu") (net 9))
 (via (at 126.6725 92.615) (size 0.6) (drill 0.3) (layers "F.Cu" "B.Cu") (free yes) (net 9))
 (segment (start 143.6265 91.99) (end 145.2265 91.99) (width 0.3) (layer "B.Cu") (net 9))
 (segment (start 126.6725 91.49) (end 130.1725 87.99) (width 0.3) (layer "B.Cu") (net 9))
 (segment (start 126.6725 92.615) (end 126.6725 91.49) (width 0.3) (layer "B.Cu") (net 9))
 (segment (start 130.1725 87.99) (end 139.6265 87.99) (width 0.3) (layer "B.Cu") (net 9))
 (segment (start 139.6265 87.99) (end 143.6265 91.99) (width 0.3) (layer "B.Cu") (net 9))
 (segment (start 131.3515 95.115) (end 130.7265 94.49) (width 0.3) (layer "F.Cu") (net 11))
 (segment (start 128.9975 95.115) (end 129.6225 94.49) (width 0.3) (layer "F.Cu") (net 11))
 (segment (start 129.6225 94.49) (end 130.7265 94.49) (width 0.3) (layer "F.Cu") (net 11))
 (segment (start 128.0265 95.115) (end 128.9975 95.115) (width 0.3) (layer "F.Cu") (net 11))
 (segment (start 136.8 94.71) (end 135.0765 94.71) (width 0.3) (layer "F.Cu") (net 3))
 (segment (start 136.8 92.15) (end 135.0765 92.15) (width 0.3) (layer "F.Cu") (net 7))
 (segment (start 136.8 89.59) (end 135.0745 89.59) (width 0.3) (layer "F.Cu") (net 13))
 (segment (start 135.0905 89.574) (end 135.0745 89.59) (width 0.3) (layer "F.Cu") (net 13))
 (segment (start 135.3305 89.574) (end 135.0765 89.32) (width 0.3) (layer "F.Cu") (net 13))
 (segment (start 133.089 98.065) (end 133.7765 97.3775) (width 0.3) (layer "F.Cu") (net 4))
 (segment (start 133.7765 97.3775) (end 133.7765 94.71) (width 0.3) (layer "F.Cu") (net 4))
 (segment (start 133.7745 92.148) (end 133.7765 92.15) (width 0.3) (layer "F.Cu") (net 4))
 (segment (start 133.7765 92.15) (end 133.7765 94.71) (width 0.3) (layer "F.Cu") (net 4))
 (segment (start 133.7745 89.59) (end 133.7745 92.148) (width 0.3) (layer "F.Cu") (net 4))
 (segment (start 141.5265 92.15) (end 141.5265 89.6) (width 0.3) (layer "F.Cu") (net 2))
 (segment (start 138.45 94.71) (end 138.45 92.15) (width 0.3) (layer "F.Cu") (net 2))
 (segment (start 138.45 92.15) (end 138.45 89.59) (width 0.3) (layer "F.Cu") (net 2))
 (segment (start 138.45 92.15) (end 141.5265 92.15) (width 0.3) (layer "F.Cu") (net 2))
 (segment (start 141.5265 94.7) (end 141.5265 92.15) (width 0.3) (layer "F.Cu") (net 2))
 (segment (start 143.5365 93.99) (end 142.8265 94.7) (width 0.3) (layer "F.Cu") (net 1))
 (segment (start 145.2265 94.2525) (end 145.2265 93.99) (width 0.3) (layer "F.Cu") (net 1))
 (segment (start 145.2265 93.99) (end 145.1265 94.09) (width 0.3) (layer "F.Cu") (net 1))
 (segment (start 145.2265 93.99) (end 143.5365 93.99) (width 0.3) (layer "F.Cu") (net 1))
 (segment (start 144.9865 89.99) (end 142.8265 92.15) (width 0.3) (layer "F.Cu") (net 14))
 (segment (start 144.8015 90.415) (end 145.2265 89.99) (width 0.3) (layer "F.Cu") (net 14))
 (segment (start 145.2265 89.99) (end 144.9865 89.99) (width 0.3) (layer "F.Cu") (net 14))
 (segment (start 145.0765 90.14) (end 145.2265 89.99) (width 0.3) (layer "B.Cu") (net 14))
 (segment (start 144.4365 87.99) (end 145.2265 87.99) (width 0.3) (layer "F.Cu") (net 12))
 (segment (start 142.8265 89.6) (end 144.4365 87.99) (width 0.3) (layer "F.Cu") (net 12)))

